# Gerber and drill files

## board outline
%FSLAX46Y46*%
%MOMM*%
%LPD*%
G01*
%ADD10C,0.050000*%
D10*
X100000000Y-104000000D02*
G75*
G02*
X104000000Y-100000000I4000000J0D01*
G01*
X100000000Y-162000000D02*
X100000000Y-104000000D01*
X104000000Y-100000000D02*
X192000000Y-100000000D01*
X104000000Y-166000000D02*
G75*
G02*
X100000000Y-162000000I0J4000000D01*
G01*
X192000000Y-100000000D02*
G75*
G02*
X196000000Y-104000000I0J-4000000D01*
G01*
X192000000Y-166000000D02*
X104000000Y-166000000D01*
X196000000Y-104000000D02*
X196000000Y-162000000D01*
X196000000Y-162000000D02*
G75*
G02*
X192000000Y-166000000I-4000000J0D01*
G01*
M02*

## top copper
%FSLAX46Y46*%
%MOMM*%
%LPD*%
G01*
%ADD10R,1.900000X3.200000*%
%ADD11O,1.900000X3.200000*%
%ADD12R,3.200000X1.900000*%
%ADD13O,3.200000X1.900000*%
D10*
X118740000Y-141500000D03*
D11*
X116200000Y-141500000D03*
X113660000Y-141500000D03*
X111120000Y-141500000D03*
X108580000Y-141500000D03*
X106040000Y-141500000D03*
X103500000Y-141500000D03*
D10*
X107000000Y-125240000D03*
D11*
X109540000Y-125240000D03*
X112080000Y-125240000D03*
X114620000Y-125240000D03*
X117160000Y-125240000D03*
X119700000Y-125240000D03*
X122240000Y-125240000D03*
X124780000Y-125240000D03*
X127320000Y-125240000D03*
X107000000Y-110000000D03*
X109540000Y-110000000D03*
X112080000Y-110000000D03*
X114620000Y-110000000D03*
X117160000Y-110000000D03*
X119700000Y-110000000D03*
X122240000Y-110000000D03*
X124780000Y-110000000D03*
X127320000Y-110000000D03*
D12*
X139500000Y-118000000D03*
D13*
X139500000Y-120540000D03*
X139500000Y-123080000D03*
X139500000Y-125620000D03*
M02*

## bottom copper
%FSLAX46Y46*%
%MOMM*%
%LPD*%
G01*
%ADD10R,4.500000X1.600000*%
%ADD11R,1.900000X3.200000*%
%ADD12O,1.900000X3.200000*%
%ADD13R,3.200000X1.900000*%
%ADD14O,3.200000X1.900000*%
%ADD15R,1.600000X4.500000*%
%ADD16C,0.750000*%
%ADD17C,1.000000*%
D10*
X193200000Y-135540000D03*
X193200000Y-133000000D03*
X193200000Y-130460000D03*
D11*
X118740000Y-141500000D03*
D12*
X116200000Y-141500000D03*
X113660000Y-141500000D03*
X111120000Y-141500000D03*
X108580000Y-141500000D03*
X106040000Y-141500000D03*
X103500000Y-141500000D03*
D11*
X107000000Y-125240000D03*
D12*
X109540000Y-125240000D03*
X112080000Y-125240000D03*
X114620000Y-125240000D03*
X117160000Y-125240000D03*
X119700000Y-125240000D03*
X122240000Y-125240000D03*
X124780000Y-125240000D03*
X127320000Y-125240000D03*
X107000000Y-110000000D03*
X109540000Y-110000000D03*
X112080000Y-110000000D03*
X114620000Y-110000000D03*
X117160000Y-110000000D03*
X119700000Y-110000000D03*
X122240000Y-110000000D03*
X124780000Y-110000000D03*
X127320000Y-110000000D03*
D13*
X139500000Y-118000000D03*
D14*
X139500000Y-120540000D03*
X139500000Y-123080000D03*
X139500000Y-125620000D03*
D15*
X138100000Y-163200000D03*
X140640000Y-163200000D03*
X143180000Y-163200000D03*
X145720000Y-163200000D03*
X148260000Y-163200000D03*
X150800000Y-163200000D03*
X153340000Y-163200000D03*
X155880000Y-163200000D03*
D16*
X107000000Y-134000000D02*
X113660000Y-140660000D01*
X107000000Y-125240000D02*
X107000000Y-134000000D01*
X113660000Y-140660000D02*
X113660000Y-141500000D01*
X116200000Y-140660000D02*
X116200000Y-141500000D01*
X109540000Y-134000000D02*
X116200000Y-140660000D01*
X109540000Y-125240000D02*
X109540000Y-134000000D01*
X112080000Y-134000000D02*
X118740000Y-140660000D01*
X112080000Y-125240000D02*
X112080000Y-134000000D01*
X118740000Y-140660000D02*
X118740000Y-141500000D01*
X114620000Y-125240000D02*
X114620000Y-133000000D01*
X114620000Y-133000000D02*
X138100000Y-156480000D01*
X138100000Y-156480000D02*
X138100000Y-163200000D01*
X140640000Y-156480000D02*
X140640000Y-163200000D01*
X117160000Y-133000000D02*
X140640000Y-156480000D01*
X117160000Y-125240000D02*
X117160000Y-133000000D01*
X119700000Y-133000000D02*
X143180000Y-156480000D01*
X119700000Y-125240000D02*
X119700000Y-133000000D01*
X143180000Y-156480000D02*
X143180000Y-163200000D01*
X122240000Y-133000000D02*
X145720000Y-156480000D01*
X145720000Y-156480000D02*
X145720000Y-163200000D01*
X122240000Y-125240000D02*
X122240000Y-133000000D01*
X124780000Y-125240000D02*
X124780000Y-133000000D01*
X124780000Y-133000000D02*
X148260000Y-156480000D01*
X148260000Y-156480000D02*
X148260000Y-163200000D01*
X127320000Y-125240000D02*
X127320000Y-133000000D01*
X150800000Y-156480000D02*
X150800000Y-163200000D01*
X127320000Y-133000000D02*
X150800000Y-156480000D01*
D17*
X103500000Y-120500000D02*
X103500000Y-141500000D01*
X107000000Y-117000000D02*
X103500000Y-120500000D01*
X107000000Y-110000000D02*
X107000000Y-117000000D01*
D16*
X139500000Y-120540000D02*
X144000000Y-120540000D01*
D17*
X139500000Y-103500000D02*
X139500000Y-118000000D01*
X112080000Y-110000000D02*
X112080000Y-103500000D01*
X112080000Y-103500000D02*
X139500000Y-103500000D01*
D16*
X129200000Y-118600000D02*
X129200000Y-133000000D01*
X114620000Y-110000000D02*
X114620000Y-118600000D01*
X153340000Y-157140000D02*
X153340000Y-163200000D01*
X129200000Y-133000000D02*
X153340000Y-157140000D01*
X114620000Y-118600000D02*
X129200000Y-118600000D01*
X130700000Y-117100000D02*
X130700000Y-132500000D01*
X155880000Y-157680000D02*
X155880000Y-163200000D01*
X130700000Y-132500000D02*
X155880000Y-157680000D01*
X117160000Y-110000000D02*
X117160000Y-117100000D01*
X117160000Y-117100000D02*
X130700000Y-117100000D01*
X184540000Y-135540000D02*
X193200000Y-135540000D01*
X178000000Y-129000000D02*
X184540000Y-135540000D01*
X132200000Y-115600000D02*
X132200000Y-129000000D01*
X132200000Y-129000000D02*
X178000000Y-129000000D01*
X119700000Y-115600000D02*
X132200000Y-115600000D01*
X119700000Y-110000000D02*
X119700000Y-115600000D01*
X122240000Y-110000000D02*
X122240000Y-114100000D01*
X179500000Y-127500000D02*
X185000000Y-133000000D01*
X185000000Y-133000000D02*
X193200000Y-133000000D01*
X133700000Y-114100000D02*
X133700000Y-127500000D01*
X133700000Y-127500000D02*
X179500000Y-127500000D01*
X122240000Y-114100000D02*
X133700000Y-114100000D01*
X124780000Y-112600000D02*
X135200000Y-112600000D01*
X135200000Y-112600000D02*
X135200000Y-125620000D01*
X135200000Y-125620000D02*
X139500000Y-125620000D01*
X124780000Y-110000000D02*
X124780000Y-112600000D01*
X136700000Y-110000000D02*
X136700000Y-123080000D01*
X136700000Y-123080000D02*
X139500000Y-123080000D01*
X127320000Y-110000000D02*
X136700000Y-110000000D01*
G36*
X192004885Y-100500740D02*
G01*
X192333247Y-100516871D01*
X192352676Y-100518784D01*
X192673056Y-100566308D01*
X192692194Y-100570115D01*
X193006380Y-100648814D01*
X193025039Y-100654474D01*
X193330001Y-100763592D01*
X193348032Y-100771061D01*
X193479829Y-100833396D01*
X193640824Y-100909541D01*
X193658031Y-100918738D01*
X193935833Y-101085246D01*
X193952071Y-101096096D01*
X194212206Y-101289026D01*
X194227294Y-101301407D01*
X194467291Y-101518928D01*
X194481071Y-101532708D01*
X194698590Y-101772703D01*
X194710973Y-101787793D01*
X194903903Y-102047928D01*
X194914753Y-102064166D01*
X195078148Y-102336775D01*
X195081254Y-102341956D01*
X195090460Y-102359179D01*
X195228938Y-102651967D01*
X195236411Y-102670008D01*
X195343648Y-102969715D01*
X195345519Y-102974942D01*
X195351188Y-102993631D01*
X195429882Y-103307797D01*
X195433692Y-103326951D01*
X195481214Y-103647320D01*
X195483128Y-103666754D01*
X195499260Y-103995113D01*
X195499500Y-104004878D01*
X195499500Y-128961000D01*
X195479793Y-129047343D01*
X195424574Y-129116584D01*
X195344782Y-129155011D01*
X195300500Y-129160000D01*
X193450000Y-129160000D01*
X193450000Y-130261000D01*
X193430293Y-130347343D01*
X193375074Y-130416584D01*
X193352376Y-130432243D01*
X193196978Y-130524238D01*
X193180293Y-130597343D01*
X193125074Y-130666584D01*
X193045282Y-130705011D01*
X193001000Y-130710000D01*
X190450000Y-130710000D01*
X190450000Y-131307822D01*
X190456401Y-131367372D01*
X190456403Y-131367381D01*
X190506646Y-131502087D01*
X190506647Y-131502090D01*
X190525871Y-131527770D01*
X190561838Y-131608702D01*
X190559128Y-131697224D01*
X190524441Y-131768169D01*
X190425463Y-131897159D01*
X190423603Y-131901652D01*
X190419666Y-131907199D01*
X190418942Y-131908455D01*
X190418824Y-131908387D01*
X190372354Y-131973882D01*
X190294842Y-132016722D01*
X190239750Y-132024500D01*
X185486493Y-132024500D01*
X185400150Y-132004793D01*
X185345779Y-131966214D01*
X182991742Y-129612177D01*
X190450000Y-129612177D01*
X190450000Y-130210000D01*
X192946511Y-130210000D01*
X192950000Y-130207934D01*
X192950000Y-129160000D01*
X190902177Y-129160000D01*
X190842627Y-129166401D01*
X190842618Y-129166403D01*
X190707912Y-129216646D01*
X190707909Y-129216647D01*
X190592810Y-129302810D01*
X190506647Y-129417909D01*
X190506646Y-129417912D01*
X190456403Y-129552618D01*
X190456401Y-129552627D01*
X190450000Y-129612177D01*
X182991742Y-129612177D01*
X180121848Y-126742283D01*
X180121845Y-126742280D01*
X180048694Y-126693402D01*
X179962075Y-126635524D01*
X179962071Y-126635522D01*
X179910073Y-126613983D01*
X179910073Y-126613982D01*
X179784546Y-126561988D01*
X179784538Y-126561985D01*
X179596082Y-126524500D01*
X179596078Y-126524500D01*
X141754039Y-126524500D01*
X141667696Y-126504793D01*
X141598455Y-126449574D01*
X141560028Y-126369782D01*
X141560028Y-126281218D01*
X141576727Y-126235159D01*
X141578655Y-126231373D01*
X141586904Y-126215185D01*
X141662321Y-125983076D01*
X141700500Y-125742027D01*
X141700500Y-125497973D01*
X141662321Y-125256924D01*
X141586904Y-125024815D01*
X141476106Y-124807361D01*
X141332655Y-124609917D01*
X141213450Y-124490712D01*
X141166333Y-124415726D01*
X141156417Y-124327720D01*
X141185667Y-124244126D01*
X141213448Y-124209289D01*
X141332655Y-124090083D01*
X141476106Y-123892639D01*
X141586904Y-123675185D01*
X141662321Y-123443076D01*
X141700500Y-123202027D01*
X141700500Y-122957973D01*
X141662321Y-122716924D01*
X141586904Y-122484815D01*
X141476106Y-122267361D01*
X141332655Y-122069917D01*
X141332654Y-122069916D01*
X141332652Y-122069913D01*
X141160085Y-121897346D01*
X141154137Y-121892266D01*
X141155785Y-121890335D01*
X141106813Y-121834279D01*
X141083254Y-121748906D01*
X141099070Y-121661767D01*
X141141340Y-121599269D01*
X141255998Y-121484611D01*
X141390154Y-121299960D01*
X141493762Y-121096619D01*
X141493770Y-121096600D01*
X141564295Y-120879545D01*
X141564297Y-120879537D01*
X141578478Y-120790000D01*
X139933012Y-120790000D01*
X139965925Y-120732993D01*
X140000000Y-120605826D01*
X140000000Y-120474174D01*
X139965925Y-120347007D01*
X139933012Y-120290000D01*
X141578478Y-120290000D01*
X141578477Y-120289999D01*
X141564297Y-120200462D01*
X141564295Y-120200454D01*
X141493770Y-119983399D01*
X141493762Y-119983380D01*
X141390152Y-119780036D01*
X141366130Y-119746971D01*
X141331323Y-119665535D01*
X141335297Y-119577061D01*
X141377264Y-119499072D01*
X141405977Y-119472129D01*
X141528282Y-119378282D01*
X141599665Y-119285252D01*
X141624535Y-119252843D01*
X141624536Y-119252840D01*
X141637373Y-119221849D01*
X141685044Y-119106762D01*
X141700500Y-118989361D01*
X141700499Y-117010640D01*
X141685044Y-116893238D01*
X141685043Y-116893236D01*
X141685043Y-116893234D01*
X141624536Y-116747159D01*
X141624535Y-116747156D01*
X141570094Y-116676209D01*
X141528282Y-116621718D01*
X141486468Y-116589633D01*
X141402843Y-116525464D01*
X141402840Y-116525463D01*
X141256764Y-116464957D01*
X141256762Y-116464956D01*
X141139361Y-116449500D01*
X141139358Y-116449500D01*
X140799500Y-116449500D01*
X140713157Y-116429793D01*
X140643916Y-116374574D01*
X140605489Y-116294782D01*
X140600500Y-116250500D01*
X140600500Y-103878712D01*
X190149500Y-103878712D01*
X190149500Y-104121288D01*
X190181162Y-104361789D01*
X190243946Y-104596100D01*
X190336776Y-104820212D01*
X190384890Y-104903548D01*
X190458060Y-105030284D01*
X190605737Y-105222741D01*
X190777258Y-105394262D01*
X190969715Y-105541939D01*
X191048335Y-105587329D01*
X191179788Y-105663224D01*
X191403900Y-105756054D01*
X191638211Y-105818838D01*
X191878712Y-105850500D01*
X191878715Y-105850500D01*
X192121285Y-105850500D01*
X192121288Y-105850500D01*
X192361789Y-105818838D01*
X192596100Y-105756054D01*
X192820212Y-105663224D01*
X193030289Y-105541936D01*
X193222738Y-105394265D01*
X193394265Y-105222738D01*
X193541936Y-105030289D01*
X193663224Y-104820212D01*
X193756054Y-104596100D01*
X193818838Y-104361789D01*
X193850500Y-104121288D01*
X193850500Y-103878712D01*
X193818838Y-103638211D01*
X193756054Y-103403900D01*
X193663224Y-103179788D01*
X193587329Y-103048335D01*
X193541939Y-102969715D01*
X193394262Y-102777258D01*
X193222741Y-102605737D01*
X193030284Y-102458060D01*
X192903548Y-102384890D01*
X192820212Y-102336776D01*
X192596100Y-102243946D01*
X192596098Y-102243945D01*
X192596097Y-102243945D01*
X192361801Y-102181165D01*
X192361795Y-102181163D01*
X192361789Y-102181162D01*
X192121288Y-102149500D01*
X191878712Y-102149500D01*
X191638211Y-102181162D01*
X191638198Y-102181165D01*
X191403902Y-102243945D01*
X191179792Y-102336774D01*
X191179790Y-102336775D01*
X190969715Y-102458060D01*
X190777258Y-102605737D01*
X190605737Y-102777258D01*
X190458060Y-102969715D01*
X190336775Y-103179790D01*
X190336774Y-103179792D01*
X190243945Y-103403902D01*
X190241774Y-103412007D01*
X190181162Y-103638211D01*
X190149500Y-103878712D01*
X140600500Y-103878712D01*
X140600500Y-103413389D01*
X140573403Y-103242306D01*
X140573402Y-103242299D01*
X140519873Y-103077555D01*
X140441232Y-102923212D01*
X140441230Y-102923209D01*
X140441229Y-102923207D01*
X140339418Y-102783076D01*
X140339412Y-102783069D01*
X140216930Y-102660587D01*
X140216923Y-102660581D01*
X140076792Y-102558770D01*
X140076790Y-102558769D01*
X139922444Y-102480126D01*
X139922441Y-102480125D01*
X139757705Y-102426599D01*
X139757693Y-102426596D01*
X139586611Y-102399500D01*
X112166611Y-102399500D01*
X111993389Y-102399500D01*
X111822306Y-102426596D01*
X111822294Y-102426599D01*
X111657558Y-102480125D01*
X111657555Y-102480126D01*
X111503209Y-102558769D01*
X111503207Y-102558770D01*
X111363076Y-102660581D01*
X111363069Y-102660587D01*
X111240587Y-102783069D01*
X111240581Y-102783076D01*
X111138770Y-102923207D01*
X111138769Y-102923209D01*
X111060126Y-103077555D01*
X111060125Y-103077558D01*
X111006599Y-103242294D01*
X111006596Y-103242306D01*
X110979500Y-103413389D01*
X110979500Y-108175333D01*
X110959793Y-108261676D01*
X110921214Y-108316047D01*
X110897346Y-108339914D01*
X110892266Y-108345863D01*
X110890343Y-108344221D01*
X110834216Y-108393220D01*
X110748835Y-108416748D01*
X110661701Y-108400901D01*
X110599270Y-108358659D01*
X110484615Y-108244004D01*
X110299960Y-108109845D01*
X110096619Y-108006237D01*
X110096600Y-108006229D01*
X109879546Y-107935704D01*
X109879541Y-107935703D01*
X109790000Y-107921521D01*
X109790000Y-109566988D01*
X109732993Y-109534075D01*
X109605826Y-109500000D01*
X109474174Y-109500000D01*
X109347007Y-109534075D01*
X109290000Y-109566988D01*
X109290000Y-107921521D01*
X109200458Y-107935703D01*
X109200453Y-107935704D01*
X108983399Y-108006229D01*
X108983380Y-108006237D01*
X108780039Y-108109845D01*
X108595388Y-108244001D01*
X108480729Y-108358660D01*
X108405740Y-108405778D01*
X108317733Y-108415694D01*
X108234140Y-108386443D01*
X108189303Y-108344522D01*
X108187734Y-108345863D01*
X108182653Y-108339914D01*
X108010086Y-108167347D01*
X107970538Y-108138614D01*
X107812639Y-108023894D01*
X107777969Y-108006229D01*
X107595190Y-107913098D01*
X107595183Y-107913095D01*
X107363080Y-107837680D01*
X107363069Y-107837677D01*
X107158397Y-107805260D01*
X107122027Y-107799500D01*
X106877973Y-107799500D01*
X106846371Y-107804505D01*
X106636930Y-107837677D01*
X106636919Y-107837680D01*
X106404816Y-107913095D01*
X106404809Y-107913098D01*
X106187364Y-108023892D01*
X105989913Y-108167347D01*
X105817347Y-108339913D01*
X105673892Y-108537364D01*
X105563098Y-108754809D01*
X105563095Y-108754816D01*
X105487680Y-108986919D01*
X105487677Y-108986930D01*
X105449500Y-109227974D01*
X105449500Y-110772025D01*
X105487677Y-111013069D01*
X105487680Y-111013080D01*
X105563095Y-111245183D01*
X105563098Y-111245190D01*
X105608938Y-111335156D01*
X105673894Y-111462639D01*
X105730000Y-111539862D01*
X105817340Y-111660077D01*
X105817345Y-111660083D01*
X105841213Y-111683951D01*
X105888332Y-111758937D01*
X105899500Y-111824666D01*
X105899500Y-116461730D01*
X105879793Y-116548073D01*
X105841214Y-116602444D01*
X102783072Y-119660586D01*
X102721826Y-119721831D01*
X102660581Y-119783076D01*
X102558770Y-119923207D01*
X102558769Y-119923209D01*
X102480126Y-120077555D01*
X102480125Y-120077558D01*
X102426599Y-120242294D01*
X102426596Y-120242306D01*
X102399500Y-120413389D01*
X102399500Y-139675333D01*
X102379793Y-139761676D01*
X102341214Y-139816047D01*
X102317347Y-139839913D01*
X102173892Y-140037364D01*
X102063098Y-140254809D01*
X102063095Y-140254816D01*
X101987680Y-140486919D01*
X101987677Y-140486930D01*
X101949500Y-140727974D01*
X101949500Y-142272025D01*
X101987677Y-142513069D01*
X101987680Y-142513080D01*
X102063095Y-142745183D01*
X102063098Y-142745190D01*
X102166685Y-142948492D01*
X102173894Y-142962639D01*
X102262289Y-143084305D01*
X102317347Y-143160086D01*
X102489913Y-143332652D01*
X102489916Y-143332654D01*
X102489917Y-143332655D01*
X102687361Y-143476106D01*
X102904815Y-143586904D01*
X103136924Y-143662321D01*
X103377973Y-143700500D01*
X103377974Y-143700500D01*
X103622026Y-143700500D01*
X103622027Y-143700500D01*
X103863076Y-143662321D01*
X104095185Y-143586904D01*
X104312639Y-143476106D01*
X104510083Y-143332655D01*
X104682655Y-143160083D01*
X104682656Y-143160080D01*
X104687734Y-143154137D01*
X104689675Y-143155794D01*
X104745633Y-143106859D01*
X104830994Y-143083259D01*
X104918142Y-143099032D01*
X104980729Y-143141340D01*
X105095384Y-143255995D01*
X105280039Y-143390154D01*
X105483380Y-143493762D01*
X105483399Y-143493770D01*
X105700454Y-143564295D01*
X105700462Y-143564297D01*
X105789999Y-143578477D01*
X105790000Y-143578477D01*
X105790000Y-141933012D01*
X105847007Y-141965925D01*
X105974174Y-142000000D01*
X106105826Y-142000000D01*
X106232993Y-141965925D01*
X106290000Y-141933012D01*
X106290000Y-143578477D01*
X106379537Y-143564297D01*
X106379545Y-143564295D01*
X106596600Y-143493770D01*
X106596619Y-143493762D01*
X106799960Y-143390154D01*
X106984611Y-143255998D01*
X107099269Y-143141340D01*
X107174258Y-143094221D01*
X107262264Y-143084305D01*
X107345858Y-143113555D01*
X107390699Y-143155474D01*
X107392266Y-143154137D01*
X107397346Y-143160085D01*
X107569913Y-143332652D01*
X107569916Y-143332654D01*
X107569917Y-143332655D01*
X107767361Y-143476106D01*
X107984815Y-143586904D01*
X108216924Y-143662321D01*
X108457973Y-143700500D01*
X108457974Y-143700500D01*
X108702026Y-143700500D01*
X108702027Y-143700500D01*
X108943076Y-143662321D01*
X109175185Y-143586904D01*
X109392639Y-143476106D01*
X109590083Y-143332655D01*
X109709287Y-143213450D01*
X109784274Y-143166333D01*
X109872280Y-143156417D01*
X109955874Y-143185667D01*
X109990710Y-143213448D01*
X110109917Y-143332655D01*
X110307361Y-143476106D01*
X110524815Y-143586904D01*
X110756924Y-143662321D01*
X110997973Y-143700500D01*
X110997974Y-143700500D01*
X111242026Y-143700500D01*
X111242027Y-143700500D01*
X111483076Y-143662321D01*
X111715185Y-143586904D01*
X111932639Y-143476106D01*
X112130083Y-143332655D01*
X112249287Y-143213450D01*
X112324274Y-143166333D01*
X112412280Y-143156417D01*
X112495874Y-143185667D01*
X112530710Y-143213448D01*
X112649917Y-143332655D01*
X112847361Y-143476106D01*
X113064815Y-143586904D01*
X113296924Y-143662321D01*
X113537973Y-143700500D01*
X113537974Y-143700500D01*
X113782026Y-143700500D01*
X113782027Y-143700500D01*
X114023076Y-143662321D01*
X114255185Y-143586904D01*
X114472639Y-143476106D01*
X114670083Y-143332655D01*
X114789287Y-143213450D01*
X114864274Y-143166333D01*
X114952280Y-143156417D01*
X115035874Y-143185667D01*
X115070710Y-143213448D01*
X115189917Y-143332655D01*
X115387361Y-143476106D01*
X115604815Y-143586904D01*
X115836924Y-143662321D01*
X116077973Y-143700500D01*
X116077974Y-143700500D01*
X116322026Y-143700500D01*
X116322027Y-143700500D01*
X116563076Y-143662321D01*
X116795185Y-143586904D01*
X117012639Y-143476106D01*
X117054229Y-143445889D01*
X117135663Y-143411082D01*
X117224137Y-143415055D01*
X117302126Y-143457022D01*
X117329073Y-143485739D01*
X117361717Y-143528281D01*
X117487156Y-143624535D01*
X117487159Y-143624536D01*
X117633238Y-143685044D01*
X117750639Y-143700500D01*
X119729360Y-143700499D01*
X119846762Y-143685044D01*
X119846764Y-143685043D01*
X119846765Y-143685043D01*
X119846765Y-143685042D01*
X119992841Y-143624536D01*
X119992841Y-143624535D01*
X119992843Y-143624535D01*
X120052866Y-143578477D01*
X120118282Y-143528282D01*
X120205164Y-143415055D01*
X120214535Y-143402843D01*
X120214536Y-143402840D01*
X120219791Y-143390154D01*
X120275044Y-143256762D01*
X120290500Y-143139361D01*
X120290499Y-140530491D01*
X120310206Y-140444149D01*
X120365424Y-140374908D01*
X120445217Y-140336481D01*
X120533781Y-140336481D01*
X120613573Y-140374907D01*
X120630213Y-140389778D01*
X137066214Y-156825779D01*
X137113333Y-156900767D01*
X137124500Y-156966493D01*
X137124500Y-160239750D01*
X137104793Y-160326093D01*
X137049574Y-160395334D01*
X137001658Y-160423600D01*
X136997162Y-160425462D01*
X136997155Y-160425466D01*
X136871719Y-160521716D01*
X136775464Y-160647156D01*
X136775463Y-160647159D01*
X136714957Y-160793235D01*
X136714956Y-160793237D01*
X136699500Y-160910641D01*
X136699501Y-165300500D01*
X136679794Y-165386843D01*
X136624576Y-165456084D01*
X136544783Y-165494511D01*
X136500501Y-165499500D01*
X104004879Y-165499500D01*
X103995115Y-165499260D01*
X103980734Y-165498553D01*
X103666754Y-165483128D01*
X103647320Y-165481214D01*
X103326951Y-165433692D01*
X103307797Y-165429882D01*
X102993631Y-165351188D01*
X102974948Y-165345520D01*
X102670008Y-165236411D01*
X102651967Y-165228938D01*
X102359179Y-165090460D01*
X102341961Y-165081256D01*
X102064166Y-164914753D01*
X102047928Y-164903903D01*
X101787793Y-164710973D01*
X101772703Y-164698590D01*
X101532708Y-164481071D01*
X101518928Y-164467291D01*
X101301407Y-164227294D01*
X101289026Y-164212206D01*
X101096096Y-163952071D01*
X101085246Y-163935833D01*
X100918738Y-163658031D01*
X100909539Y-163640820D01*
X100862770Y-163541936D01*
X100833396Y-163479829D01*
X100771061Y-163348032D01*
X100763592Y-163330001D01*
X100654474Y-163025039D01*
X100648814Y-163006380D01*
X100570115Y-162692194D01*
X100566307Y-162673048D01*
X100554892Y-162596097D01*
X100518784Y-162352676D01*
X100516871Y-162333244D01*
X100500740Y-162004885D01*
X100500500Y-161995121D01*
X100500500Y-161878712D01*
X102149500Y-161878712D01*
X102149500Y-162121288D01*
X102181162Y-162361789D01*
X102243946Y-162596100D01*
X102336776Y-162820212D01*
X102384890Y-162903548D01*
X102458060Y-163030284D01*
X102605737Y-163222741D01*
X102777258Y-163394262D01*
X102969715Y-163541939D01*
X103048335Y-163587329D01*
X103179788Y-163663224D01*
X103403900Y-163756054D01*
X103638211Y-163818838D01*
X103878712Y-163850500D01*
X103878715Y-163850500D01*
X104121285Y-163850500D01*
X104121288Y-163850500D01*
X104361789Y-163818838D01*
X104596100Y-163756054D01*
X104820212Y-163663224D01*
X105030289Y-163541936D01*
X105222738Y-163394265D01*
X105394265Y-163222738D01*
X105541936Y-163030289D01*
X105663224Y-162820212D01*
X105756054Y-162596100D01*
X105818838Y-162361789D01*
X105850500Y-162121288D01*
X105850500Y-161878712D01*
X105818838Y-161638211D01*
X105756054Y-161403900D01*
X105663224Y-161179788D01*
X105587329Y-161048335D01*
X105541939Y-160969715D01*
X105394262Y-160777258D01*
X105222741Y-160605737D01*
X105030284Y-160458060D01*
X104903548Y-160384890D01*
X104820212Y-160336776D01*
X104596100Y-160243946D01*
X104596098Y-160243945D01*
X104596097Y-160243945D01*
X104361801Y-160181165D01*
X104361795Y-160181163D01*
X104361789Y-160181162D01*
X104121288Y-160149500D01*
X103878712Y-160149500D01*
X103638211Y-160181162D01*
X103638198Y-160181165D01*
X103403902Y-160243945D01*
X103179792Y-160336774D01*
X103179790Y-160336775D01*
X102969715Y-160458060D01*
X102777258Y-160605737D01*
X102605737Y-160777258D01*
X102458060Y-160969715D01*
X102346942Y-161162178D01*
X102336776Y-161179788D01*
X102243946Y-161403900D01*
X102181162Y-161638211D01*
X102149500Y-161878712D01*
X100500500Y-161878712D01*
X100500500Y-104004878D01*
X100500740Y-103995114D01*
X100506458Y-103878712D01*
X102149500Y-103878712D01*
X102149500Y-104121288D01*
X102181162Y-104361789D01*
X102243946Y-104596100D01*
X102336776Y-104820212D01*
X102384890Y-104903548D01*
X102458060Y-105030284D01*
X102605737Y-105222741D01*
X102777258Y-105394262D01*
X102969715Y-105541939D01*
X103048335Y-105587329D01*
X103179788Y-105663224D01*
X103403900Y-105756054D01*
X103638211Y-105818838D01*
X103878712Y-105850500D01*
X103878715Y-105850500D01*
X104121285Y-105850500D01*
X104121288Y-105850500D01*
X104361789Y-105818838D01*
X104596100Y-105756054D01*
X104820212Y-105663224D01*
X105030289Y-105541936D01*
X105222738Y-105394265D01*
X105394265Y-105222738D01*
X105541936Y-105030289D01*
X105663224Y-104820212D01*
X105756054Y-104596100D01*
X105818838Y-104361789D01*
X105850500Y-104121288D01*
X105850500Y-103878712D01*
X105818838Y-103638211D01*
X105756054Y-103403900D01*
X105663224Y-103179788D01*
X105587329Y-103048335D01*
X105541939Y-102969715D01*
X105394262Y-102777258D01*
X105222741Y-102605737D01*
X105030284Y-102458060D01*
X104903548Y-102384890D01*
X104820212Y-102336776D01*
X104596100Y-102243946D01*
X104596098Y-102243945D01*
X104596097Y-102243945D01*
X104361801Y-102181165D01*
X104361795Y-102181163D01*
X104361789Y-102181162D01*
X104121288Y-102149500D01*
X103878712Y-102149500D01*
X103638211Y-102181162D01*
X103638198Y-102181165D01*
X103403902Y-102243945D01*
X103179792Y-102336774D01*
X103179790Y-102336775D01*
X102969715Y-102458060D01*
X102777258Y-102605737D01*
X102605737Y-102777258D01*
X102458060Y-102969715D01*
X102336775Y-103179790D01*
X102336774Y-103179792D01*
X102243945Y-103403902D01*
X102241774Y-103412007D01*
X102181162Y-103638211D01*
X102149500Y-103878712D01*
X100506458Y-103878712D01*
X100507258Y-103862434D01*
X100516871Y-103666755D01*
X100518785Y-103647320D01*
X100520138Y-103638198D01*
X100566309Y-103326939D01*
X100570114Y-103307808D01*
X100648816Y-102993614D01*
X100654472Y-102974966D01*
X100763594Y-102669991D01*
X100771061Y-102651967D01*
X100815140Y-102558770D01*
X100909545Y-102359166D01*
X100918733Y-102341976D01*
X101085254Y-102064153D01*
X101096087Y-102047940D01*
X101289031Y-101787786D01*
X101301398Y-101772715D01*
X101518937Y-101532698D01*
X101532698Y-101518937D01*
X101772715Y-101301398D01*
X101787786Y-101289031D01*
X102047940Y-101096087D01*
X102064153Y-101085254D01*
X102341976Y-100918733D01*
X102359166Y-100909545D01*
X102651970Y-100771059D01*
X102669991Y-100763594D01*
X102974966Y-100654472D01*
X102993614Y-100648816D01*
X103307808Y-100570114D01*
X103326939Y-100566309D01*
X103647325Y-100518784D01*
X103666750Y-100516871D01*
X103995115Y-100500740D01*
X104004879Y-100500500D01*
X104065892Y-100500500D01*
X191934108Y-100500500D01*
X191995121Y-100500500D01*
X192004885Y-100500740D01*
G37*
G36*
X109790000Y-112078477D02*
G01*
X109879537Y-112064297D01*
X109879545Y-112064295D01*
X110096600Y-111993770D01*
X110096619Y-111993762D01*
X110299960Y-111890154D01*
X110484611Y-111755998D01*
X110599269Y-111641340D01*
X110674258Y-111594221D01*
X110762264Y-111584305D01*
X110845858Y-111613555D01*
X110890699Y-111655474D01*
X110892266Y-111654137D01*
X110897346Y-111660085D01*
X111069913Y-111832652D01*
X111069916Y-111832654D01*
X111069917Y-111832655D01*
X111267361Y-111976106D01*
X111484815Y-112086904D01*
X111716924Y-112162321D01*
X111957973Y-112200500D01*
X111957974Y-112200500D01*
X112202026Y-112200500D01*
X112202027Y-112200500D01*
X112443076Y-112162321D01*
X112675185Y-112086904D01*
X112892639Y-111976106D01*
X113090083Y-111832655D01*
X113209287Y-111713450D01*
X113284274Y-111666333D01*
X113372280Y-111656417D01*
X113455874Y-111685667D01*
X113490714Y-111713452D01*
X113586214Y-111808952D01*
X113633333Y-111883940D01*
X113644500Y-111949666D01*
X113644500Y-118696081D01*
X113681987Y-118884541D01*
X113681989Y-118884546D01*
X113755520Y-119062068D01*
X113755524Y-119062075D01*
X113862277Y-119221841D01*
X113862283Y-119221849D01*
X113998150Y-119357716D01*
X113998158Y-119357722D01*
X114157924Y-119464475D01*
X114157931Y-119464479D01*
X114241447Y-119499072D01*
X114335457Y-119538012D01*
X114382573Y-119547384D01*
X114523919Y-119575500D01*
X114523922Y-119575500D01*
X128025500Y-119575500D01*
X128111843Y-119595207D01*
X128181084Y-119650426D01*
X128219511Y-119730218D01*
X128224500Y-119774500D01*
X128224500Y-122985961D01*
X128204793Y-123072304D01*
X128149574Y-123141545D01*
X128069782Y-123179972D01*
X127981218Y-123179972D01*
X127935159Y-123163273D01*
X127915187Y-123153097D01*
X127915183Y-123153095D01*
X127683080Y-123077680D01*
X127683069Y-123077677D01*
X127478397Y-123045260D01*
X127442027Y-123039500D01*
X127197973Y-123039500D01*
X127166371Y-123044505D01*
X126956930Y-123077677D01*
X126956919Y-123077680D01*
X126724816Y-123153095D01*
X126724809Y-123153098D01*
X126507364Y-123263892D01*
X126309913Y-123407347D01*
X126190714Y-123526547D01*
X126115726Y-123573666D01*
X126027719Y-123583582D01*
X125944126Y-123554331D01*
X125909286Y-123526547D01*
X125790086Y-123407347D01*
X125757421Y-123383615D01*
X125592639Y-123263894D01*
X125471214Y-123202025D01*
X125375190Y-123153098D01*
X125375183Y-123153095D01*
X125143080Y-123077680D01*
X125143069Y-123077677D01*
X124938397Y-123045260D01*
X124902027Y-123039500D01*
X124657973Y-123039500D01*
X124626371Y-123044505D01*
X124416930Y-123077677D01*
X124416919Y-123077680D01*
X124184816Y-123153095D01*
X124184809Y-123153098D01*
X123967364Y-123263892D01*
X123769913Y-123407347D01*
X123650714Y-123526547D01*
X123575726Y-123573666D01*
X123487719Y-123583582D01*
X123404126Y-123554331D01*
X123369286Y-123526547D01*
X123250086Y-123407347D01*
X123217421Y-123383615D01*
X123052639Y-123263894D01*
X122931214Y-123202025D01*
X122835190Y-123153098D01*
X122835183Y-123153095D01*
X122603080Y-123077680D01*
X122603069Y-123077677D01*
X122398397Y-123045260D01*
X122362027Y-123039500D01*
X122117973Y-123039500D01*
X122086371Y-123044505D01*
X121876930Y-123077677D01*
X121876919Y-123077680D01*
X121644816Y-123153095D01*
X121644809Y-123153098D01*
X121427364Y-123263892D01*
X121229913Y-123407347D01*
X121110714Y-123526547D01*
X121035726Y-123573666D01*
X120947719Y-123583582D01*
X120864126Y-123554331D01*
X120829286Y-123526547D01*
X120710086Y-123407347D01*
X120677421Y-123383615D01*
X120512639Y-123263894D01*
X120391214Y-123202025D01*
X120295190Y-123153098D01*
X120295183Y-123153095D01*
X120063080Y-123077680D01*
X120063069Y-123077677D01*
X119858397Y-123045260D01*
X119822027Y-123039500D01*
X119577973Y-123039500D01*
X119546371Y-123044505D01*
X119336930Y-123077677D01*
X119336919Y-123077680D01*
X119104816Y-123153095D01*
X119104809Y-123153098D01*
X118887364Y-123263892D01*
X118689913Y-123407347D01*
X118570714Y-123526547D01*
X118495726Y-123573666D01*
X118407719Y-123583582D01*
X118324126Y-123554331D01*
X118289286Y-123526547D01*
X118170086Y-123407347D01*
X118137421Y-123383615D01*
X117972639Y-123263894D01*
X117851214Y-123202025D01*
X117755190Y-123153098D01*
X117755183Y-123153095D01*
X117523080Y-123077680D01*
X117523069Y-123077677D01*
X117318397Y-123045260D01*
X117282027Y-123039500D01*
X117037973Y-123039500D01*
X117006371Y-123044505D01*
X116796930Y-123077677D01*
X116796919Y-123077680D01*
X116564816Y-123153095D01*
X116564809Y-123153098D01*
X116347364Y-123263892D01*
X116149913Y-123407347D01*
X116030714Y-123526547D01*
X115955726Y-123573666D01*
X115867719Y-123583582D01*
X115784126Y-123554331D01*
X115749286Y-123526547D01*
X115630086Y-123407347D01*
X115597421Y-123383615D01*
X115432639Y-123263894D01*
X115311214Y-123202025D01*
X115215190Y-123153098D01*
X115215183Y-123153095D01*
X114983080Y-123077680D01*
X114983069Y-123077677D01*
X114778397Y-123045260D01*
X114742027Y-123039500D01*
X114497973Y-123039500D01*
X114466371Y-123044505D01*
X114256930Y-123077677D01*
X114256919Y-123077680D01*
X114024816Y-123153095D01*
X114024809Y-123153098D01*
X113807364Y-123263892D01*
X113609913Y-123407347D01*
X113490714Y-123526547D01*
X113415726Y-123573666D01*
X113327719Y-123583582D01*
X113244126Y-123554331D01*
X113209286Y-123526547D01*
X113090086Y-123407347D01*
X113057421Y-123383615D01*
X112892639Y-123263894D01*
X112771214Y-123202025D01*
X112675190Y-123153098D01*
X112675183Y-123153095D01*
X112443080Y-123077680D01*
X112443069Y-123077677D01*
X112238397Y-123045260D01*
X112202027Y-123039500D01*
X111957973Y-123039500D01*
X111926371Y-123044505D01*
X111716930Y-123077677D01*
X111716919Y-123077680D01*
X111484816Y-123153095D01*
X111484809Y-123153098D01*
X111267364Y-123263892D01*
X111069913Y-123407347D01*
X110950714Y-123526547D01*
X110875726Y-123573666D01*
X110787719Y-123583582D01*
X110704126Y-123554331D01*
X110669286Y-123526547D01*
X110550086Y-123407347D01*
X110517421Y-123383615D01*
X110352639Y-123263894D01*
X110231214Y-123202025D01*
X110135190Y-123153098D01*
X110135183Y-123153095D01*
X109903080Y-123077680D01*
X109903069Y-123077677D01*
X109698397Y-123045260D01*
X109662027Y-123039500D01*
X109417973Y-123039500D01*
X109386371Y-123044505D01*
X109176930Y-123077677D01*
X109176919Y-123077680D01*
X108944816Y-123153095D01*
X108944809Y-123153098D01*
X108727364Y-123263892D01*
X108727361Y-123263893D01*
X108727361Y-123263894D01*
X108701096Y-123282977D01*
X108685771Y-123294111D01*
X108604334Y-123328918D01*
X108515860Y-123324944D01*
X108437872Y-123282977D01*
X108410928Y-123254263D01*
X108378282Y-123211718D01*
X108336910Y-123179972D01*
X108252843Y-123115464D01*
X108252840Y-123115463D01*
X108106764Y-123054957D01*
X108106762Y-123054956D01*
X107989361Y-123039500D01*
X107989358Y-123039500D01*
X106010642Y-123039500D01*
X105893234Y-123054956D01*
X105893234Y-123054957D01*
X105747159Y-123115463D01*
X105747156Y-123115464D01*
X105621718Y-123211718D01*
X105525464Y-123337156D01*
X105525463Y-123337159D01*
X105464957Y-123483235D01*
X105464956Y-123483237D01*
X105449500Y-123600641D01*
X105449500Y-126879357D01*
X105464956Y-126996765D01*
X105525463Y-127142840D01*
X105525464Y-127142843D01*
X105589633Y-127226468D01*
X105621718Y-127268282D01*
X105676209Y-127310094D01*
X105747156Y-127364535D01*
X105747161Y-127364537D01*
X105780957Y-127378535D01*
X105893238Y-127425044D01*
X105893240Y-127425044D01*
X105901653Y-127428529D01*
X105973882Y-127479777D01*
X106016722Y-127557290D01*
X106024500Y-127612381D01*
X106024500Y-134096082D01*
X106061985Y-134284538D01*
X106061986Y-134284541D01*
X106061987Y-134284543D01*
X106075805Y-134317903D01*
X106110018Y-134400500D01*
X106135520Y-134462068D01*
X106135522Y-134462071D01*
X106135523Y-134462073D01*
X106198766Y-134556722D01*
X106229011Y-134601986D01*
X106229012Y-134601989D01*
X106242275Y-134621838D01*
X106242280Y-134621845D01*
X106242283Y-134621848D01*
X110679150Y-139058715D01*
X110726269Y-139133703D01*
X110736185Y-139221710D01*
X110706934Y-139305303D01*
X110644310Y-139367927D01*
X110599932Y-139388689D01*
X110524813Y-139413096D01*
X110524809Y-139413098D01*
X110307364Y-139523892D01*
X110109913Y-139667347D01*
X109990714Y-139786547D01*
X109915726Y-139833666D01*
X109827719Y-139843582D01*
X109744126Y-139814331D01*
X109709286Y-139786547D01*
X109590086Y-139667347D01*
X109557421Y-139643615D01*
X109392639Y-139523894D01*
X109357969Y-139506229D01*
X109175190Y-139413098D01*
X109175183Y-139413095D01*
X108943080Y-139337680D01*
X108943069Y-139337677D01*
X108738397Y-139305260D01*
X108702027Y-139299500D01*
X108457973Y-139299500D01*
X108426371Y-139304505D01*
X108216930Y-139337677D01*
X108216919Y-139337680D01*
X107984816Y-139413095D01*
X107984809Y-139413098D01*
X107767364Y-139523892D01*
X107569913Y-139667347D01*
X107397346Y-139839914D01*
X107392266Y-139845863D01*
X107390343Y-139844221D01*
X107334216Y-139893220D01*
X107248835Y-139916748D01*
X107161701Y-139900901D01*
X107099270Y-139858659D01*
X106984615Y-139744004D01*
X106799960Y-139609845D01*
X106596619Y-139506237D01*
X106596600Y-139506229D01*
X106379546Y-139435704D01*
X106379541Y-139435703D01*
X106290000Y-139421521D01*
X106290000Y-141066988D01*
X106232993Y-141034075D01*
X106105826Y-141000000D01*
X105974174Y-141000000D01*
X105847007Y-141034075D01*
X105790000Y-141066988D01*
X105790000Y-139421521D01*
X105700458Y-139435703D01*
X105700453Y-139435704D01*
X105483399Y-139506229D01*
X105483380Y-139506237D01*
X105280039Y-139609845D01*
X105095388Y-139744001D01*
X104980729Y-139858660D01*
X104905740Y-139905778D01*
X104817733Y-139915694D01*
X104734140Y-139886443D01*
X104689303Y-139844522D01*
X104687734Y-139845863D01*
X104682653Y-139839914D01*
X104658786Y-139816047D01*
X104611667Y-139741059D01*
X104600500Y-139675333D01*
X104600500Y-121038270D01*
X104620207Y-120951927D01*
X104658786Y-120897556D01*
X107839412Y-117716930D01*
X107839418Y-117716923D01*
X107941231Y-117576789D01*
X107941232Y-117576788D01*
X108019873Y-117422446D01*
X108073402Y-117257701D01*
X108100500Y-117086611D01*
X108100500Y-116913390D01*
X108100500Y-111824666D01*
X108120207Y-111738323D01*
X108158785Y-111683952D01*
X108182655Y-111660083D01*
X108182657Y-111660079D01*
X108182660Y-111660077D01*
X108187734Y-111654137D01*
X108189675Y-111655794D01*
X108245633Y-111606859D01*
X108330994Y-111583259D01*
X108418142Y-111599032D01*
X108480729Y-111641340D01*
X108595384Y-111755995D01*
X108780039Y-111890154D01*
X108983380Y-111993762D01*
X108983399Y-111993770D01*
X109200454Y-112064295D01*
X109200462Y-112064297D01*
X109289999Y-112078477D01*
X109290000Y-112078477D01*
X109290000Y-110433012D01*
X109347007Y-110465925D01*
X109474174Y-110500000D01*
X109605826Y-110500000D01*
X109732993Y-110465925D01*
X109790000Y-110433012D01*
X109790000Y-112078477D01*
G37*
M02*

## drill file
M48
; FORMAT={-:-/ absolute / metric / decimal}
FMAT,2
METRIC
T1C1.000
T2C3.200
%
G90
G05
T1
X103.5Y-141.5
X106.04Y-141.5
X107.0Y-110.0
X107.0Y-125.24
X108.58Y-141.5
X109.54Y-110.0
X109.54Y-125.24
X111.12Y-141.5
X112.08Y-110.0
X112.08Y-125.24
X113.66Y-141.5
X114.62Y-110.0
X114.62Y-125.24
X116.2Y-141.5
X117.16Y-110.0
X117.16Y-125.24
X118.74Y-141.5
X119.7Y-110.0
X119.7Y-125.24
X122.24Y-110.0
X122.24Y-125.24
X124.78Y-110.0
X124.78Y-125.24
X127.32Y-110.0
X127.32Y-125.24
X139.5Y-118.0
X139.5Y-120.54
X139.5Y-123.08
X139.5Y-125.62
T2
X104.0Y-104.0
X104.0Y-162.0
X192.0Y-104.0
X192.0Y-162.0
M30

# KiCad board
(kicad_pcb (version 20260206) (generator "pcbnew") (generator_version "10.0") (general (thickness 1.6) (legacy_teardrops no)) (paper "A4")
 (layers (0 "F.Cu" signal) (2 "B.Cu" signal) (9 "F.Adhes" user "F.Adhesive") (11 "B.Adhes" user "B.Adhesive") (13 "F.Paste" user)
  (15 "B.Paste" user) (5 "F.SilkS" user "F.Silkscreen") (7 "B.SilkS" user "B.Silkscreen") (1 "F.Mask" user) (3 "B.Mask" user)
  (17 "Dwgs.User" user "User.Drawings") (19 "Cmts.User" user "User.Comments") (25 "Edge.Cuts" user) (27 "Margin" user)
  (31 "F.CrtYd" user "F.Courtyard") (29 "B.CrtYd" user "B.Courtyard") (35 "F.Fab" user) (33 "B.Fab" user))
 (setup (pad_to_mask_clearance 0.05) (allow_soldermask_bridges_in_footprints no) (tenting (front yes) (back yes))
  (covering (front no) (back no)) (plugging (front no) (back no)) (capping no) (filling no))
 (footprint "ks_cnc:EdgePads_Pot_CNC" (layer "F.Cu") (at 193.2 135.54 90)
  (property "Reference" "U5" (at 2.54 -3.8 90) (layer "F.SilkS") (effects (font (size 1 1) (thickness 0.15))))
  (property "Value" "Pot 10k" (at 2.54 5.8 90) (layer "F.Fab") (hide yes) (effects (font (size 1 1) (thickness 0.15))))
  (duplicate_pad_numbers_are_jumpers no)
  (pad "1" smd rect (at 0 0 90) (size 1.6 4.5) (layers "B.Cu" "B.Mask") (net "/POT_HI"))
  (pad "2" smd rect (at 2.54 0 90) (size 1.6 4.5) (layers "B.Cu" "B.Mask") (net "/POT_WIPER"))
  (pad "3" smd rect (at 5.08 0 90) (size 1.6 4.5) (layers "B.Cu" "B.Mask") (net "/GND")))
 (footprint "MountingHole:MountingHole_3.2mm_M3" (layer "F.Cu") (at 104 104)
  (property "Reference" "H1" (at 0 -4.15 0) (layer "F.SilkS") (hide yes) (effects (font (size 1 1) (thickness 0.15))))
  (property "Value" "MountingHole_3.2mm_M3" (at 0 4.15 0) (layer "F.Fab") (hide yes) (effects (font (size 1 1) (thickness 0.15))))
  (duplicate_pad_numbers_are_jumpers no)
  (pad "" np_thru_hole circle (at 0 0) (size 3.2 3.2) (drill 3.2) (layers "*.Cu" "*.Mask")))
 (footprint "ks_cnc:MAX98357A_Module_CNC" (layer "F.Cu") (at 118.74 141.5 -90)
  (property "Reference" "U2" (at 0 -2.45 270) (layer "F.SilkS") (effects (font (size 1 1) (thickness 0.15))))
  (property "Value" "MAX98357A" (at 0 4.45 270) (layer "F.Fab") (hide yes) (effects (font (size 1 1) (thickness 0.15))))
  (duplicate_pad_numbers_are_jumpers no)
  (pad "1" thru_hole rect (at 0 0 270) (size 3.2 1.9) (drill 1) (layers "*.Cu" "B.Mask") (remove_unused_layers no) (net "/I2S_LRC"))
  (pad "2" thru_hole oval (at 0 2.54 270) (size 3.2 1.9) (drill 1) (layers "*.Cu" "B.Mask") (remove_unused_layers no) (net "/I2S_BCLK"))
  (pad "3" thru_hole oval (at 0 5.08 270) (size 3.2 1.9) (drill 1) (layers "*.Cu" "B.Mask") (remove_unused_layers no) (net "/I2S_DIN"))
  (pad "4" thru_hole oval (at 0 7.62 270) (size 3.2 1.9) (drill 1) (layers "*.Cu" "B.Mask") (remove_unused_layers no)
   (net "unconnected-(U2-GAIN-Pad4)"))
  (pad "5" thru_hole oval (at 0 10.16 270) (size 3.2 1.9) (drill 1) (layers "*.Cu" "B.Mask") (remove_unused_layers no)
   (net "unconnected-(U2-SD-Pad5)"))
  (pad "6" thru_hole oval (at 0 12.7 270) (size 3.2 1.9) (drill 1) (layers "*.Cu" "B.Mask") (remove_unused_layers no) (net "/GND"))
  (pad "7" thru_hole oval (at 0 15.24 270) (size 3.2 1.9) (drill 1) (layers "*.Cu" "B.Mask") (remove_unused_layers no) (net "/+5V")))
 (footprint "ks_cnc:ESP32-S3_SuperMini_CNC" (layer "F.Cu") (at 107 125.24 90)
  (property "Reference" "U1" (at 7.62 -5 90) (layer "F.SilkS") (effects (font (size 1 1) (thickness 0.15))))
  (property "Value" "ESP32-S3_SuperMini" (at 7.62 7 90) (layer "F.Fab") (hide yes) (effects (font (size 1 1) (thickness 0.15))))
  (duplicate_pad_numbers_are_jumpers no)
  (pad "1" thru_hole rect (at 0 0 90) (size 3.2 1.9) (drill 1) (layers "*.Cu" "B.Mask") (remove_unused_layers no) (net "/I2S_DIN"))
  (pad "2" thru_hole oval (at 0 2.54 90) (size 3.2 1.9) (drill 1) (layers "*.Cu" "B.Mask") (remove_unused_layers no) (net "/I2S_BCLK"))
  (pad "3" thru_hole oval (at 0 5.08 90) (size 3.2 1.9) (drill 1) (layers "*.Cu" "B.Mask") (remove_unused_layers no) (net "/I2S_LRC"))
  (pad "4" thru_hole oval (at 0 7.62 90) (size 3.2 1.9) (drill 1) (layers "*.Cu" "B.Mask") (remove_unused_layers no) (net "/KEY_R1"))
  (pad "5" thru_hole oval (at 0 10.16 90) (size 3.2 1.9) (drill 1) (layers "*.Cu" "B.Mask") (remove_unused_layers no) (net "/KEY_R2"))
  (pad "6" thru_hole oval (at 0 12.7 90) (size 3.2 1.9) (drill 1) (layers "*.Cu" "B.Mask") (remove_unused_layers no) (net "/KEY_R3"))
  (pad "7" thru_hole oval (at 0 15.24 90) (size 3.2 1.9) (drill 1) (layers "*.Cu" "B.Mask") (remove_unused_layers no) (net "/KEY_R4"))
  (pad "8" thru_hole oval (at 0 17.78 90) (size 3.2 1.9) (drill 1) (layers "*.Cu" "B.Mask") (remove_unused_layers no) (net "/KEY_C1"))
  (pad "9" thru_hole oval (at 0 20.32 90) (size 3.2 1.9) (drill 1) (layers "*.Cu" "B.Mask") (remove_unused_layers no) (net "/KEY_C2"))
  (pad "10" thru_hole oval (at 15.24 0 90) (size 3.2 1.9) (drill 1) (layers "*.Cu" "B.Mask") (remove_unused_layers no) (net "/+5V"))
  (pad "11" thru_hole oval (at 15.24 2.54 90) (size 3.2 1.9) (drill 1) (layers "*.Cu" "B.Mask") (remove_unused_layers no) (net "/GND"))
  (pad "12" thru_hole oval (at 15.24 5.08 90) (size 3.2 1.9) (drill 1) (layers "*.Cu" "B.Mask") (remove_unused_layers no) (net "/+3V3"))
  (pad "13" thru_hole oval (at 15.24 7.62 90) (size 3.2 1.9) (drill 1) (layers "*.Cu" "B.Mask") (remove_unused_layers no) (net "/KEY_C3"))
  (pad "14" thru_hole oval (at 15.24 10.16 90) (size 3.2 1.9) (drill 1) (layers "*.Cu" "B.Mask") (remove_unused_layers no) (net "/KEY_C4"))
  (pad "15" thru_hole oval (at 15.24 12.7 90) (size 3.2 1.9) (drill 1) (layers "*.Cu" "B.Mask") (remove_unused_layers no) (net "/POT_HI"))
  (pad "16" thru_hole oval (at 15.24 15.24 90) (size 3.2 1.9) (drill 1) (layers "*.Cu" "B.Mask") (remove_unused_layers no)
   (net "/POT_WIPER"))
  (pad "17" thru_hole oval (at 15.24 17.78 90) (size 3.2 1.9) (drill 1) (layers "*.Cu" "B.Mask") (remove_unused_layers no) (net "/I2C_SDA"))
  (pad "18" thru_hole oval (at 15.24 20.32 90) (size 3.2 1.9) (drill 1) (layers "*.Cu" "B.Mask") (remove_unused_layers no) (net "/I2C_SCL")))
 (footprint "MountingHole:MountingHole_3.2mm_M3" (layer "F.Cu") (at 192 104)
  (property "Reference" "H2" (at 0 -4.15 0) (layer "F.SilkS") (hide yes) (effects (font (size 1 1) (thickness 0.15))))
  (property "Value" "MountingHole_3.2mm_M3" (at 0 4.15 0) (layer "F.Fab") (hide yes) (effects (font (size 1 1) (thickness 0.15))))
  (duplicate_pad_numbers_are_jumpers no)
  (pad "" np_thru_hole circle (at 0 0) (size 3.2 3.2) (drill 3.2) (layers "*.Cu" "*.Mask")))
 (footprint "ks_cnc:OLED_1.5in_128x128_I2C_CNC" (layer "F.Cu") (at 139.5 118)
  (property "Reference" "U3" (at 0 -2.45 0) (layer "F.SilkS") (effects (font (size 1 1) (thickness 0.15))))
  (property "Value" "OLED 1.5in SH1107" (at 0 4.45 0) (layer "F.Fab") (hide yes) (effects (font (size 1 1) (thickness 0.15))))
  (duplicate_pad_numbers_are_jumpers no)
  (pad "1" thru_hole rect (at 0 0) (size 3.2 1.9) (drill 1) (layers "*.Cu" "B.Mask") (remove_unused_layers no) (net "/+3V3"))
  (pad "2" thru_hole oval (at 0 2.54) (size 3.2 1.9) (drill 1) (layers "*.Cu" "B.Mask") (remove_unused_layers no) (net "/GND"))
  (pad "3" thru_hole oval (at 0 5.08) (size 3.2 1.9) (drill 1) (layers "*.Cu" "B.Mask") (remove_unused_layers no) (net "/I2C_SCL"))
  (pad "4" thru_hole oval (at 0 7.62) (size 3.2 1.9) (drill 1) (layers "*.Cu" "B.Mask") (remove_unused_layers no) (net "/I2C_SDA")))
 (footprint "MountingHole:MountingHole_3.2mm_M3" (layer "F.Cu") (at 104 162)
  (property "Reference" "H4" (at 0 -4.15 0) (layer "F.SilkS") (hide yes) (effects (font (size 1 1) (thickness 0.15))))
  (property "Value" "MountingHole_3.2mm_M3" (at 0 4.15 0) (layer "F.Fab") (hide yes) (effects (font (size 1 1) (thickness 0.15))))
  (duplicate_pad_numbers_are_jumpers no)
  (pad "" np_thru_hole circle (at 0 0) (size 3.2 3.2) (drill 3.2) (layers "*.Cu" "*.Mask")))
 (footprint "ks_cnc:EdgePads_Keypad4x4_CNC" (layer "F.Cu") (at 138.1 163.2)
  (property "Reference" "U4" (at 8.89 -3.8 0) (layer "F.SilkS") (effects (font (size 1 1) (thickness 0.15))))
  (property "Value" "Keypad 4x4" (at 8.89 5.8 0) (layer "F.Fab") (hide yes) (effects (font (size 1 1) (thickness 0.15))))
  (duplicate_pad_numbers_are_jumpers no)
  (pad "1" smd rect (at 0 0) (size 1.6 4.5) (layers "B.Cu" "B.Mask") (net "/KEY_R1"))
  (pad "2" smd rect (at 2.54 0) (size 1.6 4.5) (layers "B.Cu" "B.Mask") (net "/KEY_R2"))
  (pad "3" smd rect (at 5.08 0) (size 1.6 4.5) (layers "B.Cu" "B.Mask") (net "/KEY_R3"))
  (pad "4" smd rect (at 7.62 0) (size 1.6 4.5) (layers "B.Cu" "B.Mask") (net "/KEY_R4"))
  (pad "5" smd rect (at 10.16 0) (size 1.6 4.5) (layers "B.Cu" "B.Mask") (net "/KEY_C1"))
  (pad "6" smd rect (at 12.7 0) (size 1.6 4.5) (layers "B.Cu" "B.Mask") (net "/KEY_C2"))
  (pad "7" smd rect (at 15.24 0) (size 1.6 4.5) (layers "B.Cu" "B.Mask") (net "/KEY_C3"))
  (pad "8" smd rect (at 17.78 0) (size 1.6 4.5) (layers "B.Cu" "B.Mask") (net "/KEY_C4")))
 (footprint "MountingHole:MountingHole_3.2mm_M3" (layer "F.Cu") (at 192 162)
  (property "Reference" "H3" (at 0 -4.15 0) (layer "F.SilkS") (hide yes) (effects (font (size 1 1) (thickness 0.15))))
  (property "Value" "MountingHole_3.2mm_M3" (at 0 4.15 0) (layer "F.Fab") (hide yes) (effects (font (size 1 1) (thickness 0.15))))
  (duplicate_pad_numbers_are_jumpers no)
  (pad "" np_thru_hole circle (at 0 0) (size 3.2 3.2) (drill 3.2) (layers "*.Cu" "*.Mask")))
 (gr_arc (start 100 104) (mid 101.171573 101.171573) (end 104 100) (stroke (width 0.05) (type default)) (layer "Edge.Cuts"))
 (gr_line (start 100 162) (end 100 104) (stroke (width 0.05) (type default)) (layer "Edge.Cuts"))
 (gr_line (start 104 100) (end 192 100) (stroke (width 0.05) (type default)) (layer "Edge.Cuts"))
 (gr_arc (start 104 166) (mid 101.171573 164.828427) (end 100 162) (stroke (width 0.05) (type default)) (layer "Edge.Cuts"))
 (gr_arc (start 192 100) (mid 194.828427 101.171573) (end 196 104) (stroke (width 0.05) (type default)) (layer "Edge.Cuts"))
 (gr_line (start 192 166) (end 104 166) (stroke (width 0.05) (type default)) (layer "Edge.Cuts"))
 (gr_line (start 196 104) (end 196 162) (stroke (width 0.05) (type default)) (layer "Edge.Cuts"))
 (gr_arc (start 196 162) (mid 194.828427 164.828427) (end 192 166) (stroke (width 0.05) (type default)) (layer "Edge.Cuts"))
 (segment (start 107 134) (end 113.66 140.66) (width 0.75) (layer "B.Cu") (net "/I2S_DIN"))
 (segment (start 107 125.24) (end 107 134) (width 0.75) (layer "B.Cu") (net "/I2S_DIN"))
 (segment (start 113.66 140.66) (end 113.66 141.5) (width 0.75) (layer "B.Cu") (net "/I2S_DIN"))
 (segment (start 116.2 140.66) (end 116.2 141.5) (width 0.75) (layer "B.Cu") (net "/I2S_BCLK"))
 (segment (start 109.54 134) (end 116.2 140.66) (width 0.75) (layer "B.Cu") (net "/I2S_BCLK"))
 (segment (start 109.54 125.24) (end 109.54 134) (width 0.75) (layer "B.Cu") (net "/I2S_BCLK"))
 (segment (start 112.08 134) (end 118.74 140.66) (width 0.75) (layer "B.Cu") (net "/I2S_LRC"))
 (segment (start 112.08 125.24) (end 112.08 134) (width 0.75) (layer "B.Cu") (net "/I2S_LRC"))
 (segment (start 118.74 140.66) (end 118.74 141.5) (width 0.75) (layer "B.Cu") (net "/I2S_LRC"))
 (segment (start 114.62 125.24) (end 114.62 133) (width 0.75) (layer "B.Cu") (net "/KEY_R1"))
 (segment (start 114.62 133) (end 138.1 156.48) (width 0.75) (layer "B.Cu") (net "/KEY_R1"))
 (segment (start 138.1 156.48) (end 138.1 163.2) (width 0.75) (layer "B.Cu") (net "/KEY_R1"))
 (segment (start 140.64 156.48) (end 140.64 163.2) (width 0.75) (layer "B.Cu") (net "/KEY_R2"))
 (segment (start 117.16 133) (end 140.64 156.48) (width 0.75) (layer "B.Cu") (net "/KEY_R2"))
 (segment (start 117.16 125.24) (end 117.16 133) (width 0.75) (layer "B.Cu") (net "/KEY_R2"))
 (segment (start 119.7 133) (end 143.18 156.48) (width 0.75) (layer "B.Cu") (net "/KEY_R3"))
 (segment (start 119.7 125.24) (end 119.7 133) (width 0.75) (layer "B.Cu") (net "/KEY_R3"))
 (segment (start 143.18 156.48) (end 143.18 163.2) (width 0.75) (layer "B.Cu") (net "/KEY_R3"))
 (segment (start 122.24 133) (end 145.72 156.48) (width 0.75) (layer "B.Cu") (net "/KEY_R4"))
 (segment (start 145.72 156.48) (end 145.72 163.2) (width 0.75) (layer "B.Cu") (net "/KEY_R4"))
 (segment (start 122.24 125.24) (end 122.24 133) (width 0.75) (layer "B.Cu") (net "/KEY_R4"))
 (segment (start 124.78 125.24) (end 124.78 133) (width 0.75) (layer "B.Cu") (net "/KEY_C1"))
 (segment (start 124.78 133) (end 148.26 156.48) (width 0.75) (layer "B.Cu") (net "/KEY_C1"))
 (segment (start 148.26 156.48) (end 148.26 163.2) (width 0.75) (layer "B.Cu") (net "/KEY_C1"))
 (segment (start 127.32 125.24) (end 127.32 133) (width 0.75) (layer "B.Cu") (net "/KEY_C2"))
 (segment (start 150.8 156.48) (end 150.8 163.2) (width 0.75) (layer "B.Cu") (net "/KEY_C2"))
 (segment (start 127.32 133) (end 150.8 156.48) (width 0.75) (layer "B.Cu") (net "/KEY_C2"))
 (segment (start 103.5 120.5) (end 103.5 141.5) (width 1) (layer "B.Cu") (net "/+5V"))
 (segment (start 107 117) (end 103.5 120.5) (width 1) (layer "B.Cu") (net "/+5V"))
 (segment (start 107 110) (end 107 117) (width 1) (layer "B.Cu") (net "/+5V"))
 (segment (start 139.5 120.54) (end 144 120.54) (width 0.75) (layer "B.Cu") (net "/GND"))
 (segment (start 139.5 103.5) (end 139.5 118) (width 1) (layer "B.Cu") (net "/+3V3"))
 (segment (start 112.08 110) (end 112.08 103.5) (width 1) (layer "B.Cu") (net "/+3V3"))
 (segment (start 112.08 103.5) (end 139.5 103.5) (width 1) (layer "B.Cu") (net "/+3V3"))
 (segment (start 129.2 118.6) (end 129.2 133) (width 0.75) (layer "B.Cu") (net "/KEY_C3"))
 (segment (start 114.62 110) (end 114.62 118.6) (width 0.75) (layer "B.Cu") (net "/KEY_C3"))
 (segment (start 153.34 157.14) (end 153.34 163.2) (width 0.75) (layer "B.Cu") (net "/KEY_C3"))
 (segment (start 129.2 133) (end 153.34 157.14) (width 0.75) (layer "B.Cu") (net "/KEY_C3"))
 (segment (start 114.62 118.6) (end 129.2 118.6) (width 0.75) (layer "B.Cu") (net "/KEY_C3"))
 (segment (start 130.7 117.1) (end 130.7 132.5) (width 0.75) (layer "B.Cu") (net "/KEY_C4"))
 (segment (start 155.88 157.68) (end 155.88 163.2) (width 0.75) (layer "B.Cu") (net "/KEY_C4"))
 (segment (start 130.7 132.5) (end 155.88 157.68) (width 0.75) (layer "B.Cu") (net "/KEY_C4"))
 (segment (start 117.16 110) (end 117.16 117.1) (width 0.75) (layer "B.Cu") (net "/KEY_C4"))
 (segment (start 117.16 117.1) (end 130.7 117.1) (width 0.75) (layer "B.Cu") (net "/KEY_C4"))
 (segment (start 184.54 135.54) (end 193.2 135.54) (width 0.75) (layer "B.Cu") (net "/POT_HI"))
 (segment (start 178 129) (end 184.54 135.54) (width 0.75) (layer "B.Cu") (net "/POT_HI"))
 (segment (start 132.2 115.6) (end 132.2 129) (width 0.75) (layer "B.Cu") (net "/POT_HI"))
 (segment (start 132.2 129) (end 178 129) (width 0.75) (layer "B.Cu") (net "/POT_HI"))
 (segment (start 119.7 115.6) (end 132.2 115.6) (width 0.75) (layer "B.Cu") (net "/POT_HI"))
 (segment (start 119.7 110) (end 119.7 115.6) (width 0.75) (layer "B.Cu") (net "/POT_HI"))
 (segment (start 122.24 110) (end 122.24 114.1) (width 0.75) (layer "B.Cu") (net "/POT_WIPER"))
 (segment (start 179.5 127.5) (end 185 133) (width 0.75) (layer "B.Cu") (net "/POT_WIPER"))
 (segment (start 185 133) (end 193.2 133) (width 0.75) (layer "B.Cu") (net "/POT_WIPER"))
 (segment (start 133.7 114.1) (end 133.7 127.5) (width 0.75) (layer "B.Cu") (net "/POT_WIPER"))
 (segment (start 133.7 127.5) (end 179.5 127.5) (width 0.75) (layer "B.Cu") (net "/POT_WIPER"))
 (segment (start 122.24 114.1) (end 133.7 114.1) (width 0.75) (layer "B.Cu") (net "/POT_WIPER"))
 (segment (start 124.78 112.6) (end 135.2 112.6) (width 0.75) (layer "B.Cu") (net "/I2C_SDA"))
 (segment (start 135.2 112.6) (end 135.2 125.62) (width 0.75) (layer "B.Cu") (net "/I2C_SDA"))
 (segment (start 135.2 125.62) (end 139.5 125.62) (width 0.75) (layer "B.Cu") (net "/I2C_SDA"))
 (segment (start 124.78 110) (end 124.78 112.6) (width 0.75) (layer "B.Cu") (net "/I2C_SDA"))
 (segment (start 136.7 110) (end 136.7 123.08) (width 0.75) (layer "B.Cu") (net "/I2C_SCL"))
 (segment (start 136.7 123.08) (end 139.5 123.08) (width 0.75) (layer "B.Cu") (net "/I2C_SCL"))
 (segment (start 127.32 110) (end 136.7 110) (width 0.75) (layer "B.Cu") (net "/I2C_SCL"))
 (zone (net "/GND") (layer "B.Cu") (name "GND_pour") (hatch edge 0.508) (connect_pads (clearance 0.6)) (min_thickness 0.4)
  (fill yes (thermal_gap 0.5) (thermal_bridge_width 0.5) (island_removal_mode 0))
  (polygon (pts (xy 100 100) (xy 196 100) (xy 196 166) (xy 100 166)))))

